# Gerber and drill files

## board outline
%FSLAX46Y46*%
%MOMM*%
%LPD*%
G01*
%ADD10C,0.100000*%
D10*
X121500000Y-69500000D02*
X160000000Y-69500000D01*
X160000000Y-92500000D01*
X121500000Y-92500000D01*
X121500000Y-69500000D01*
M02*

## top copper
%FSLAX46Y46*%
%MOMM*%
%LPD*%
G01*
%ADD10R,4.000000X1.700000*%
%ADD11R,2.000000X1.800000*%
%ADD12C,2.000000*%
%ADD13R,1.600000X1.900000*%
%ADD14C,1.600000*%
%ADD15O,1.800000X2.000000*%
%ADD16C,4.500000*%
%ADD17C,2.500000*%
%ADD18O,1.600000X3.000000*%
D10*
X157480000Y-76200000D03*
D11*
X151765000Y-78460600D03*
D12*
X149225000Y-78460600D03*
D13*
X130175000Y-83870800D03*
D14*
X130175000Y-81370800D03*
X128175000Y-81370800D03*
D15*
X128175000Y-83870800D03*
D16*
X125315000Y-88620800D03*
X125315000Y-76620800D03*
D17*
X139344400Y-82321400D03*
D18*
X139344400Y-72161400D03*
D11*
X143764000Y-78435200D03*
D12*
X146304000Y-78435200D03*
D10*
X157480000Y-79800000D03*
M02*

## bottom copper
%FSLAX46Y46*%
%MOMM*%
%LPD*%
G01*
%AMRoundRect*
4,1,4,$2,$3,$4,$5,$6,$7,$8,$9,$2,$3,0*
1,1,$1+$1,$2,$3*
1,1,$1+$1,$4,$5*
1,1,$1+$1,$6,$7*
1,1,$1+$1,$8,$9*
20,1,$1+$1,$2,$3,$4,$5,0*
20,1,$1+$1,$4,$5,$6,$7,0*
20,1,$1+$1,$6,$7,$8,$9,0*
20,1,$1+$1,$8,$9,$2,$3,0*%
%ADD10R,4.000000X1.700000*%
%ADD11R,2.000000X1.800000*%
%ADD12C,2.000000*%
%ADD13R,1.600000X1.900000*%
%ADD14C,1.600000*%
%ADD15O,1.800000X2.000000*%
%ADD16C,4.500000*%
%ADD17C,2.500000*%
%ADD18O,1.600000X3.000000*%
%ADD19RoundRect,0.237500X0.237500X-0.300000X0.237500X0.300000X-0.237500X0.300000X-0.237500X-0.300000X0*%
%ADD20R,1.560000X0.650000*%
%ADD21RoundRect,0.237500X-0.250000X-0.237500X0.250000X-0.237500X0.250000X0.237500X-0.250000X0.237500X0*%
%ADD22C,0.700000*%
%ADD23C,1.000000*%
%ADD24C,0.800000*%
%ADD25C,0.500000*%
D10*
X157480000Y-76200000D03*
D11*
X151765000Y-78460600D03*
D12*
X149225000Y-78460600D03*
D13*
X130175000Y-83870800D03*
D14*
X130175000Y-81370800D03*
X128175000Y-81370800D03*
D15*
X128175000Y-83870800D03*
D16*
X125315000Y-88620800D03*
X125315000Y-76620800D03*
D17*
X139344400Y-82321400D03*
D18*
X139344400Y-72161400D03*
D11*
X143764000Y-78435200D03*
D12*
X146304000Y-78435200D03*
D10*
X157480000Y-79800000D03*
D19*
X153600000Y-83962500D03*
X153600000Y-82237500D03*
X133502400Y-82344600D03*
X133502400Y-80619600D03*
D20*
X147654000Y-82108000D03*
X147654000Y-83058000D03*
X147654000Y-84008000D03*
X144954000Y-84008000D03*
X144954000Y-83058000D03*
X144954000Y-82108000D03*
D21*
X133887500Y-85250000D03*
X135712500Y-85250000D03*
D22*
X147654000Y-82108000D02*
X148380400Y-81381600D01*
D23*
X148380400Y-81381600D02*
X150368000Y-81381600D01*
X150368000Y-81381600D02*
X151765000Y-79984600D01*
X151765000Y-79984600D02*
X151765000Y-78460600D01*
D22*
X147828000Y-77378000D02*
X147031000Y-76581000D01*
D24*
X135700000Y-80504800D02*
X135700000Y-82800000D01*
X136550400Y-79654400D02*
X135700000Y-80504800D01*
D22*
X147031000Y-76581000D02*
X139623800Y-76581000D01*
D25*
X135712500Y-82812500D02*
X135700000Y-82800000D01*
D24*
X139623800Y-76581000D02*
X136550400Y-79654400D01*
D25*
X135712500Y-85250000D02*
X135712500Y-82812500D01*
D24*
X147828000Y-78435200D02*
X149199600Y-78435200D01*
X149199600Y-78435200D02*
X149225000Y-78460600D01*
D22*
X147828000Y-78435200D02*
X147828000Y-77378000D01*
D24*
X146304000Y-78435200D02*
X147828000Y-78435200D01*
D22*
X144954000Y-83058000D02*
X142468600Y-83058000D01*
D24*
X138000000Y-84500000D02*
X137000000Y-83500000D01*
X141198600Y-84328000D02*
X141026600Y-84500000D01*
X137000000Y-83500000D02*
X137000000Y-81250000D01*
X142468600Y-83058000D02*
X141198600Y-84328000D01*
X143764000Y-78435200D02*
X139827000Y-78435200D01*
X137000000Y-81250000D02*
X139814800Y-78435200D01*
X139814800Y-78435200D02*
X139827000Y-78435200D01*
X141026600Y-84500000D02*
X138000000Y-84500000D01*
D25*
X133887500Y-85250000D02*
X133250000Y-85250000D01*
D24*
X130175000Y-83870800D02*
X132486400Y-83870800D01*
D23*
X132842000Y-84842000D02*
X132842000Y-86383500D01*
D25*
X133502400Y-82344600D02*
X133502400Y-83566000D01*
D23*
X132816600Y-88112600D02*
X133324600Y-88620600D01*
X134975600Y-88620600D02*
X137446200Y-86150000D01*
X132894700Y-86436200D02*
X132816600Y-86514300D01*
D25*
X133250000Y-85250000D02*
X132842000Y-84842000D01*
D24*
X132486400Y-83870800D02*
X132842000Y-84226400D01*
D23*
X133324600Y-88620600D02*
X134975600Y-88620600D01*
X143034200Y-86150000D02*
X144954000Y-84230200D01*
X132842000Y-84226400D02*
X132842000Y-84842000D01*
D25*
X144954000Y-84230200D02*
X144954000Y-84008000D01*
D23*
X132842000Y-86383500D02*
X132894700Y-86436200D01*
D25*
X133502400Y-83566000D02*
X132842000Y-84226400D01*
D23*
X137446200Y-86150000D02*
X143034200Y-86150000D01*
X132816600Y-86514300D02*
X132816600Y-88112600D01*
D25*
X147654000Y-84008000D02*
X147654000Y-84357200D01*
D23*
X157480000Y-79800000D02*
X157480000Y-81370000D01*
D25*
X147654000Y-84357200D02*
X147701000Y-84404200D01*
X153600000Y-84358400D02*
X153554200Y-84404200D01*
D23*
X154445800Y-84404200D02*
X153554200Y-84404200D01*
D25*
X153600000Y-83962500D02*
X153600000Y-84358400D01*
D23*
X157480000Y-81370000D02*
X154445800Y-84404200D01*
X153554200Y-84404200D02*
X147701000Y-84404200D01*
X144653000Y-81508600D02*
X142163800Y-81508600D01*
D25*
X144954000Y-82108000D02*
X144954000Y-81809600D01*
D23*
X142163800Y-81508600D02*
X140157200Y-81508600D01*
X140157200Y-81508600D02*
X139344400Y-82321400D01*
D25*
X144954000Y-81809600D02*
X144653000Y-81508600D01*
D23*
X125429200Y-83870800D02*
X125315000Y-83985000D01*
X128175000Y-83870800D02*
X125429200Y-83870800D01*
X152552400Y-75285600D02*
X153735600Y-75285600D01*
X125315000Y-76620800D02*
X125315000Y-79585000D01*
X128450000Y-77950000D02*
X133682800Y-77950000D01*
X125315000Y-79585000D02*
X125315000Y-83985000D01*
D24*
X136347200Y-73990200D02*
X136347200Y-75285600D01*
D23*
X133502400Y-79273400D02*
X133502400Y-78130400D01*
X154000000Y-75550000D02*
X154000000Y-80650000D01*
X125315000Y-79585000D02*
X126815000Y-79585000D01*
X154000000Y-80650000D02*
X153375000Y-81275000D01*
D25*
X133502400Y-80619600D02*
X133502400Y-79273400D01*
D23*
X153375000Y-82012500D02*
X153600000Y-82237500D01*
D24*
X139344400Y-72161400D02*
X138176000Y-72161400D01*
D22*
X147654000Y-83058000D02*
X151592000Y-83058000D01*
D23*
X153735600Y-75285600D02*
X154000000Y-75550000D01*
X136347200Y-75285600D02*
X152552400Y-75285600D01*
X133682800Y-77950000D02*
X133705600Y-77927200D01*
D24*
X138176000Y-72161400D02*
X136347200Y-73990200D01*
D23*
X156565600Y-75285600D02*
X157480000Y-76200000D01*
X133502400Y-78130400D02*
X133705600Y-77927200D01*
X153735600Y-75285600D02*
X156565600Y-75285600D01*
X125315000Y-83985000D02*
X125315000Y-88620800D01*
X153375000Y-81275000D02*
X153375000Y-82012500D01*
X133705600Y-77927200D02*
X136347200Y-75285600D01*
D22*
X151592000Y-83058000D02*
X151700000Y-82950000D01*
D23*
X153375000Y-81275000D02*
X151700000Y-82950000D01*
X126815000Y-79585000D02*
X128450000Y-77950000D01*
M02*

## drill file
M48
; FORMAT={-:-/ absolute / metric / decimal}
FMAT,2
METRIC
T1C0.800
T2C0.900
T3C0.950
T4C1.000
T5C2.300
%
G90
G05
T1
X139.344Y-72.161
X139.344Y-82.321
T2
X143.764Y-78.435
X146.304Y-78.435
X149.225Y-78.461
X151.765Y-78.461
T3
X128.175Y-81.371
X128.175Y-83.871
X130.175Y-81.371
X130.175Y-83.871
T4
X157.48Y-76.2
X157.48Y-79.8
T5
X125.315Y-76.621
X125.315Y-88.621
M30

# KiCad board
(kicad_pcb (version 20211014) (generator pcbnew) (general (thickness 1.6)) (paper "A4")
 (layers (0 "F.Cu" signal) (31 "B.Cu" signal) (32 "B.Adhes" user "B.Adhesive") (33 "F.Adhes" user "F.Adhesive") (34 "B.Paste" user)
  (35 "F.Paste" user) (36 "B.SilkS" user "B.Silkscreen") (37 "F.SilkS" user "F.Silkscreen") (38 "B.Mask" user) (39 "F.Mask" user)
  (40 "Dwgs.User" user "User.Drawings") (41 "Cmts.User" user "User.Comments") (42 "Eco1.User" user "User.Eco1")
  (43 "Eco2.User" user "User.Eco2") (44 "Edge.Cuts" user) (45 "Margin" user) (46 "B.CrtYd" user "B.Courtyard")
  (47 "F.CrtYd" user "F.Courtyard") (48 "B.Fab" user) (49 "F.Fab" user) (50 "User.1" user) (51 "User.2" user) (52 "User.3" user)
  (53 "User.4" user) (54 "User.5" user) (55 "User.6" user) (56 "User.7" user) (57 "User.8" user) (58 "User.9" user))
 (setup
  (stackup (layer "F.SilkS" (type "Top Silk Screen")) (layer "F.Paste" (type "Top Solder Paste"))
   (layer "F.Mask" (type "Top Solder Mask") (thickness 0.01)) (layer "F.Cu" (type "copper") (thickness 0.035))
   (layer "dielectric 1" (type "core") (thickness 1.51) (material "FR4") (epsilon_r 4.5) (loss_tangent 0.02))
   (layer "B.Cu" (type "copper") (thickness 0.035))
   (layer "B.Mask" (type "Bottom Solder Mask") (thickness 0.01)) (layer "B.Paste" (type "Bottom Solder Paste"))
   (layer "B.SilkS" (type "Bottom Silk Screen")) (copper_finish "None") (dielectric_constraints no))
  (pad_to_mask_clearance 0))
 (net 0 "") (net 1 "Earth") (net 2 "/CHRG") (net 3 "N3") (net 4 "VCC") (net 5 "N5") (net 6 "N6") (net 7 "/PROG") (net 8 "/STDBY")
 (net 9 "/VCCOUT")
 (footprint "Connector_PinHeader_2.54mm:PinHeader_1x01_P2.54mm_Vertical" (layer "F.Cu") (at 157.48 76.2)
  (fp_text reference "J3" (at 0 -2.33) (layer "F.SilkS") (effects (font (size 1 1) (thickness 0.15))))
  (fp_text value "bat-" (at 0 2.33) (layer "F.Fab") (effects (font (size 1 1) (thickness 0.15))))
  (pad "1" thru_hole rect (at 0 0) (size 4 1.7) (drill 1) (layers *.Cu) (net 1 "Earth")))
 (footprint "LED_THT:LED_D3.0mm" (layer "F.Cu") (at 151.765 78.4606 180)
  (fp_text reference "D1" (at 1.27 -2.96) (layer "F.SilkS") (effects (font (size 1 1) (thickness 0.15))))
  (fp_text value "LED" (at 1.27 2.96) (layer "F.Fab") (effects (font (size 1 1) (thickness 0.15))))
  (pad "1" thru_hole rect (at 0 0 180) (size 2 1.8) (drill 0.9) (layers *.Cu *.Mask) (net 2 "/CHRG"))
  (pad "2" thru_hole circle (at 2.54 0 180) (size 2 2) (drill 0.9) (layers *.Cu *.Mask) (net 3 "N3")))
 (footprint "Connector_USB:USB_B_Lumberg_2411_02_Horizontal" (layer "F.Cu") (at 130.175 83.8708 180)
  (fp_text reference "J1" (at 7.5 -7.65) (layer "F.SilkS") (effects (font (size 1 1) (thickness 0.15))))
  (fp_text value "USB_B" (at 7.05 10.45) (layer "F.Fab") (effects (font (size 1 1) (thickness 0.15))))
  (pad "1" thru_hole rect (at 0 0 270) (size 1.9 1.6) (drill 0.95) (layers *.Cu *.Mask) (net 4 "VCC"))
  (pad "2" thru_hole circle (at 0 2.5 270) (size 1.6 1.6) (drill 0.95) (layers *.Cu *.Mask) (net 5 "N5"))
  (pad "3" thru_hole circle (at 2 2.5 270) (size 1.6 1.6) (drill 0.95) (layers *.Cu *.Mask) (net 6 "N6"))
  (pad "4" thru_hole oval (at 2 0 270) (size 2 1.8) (drill 0.95) (layers *.Cu *.Mask) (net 1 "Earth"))
  (pad "5" thru_hole circle (at 4.86 -4.75 270) (size 4.5 4.5) (drill 2.3) (layers *.Cu *.Mask) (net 1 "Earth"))
  (pad "5" thru_hole circle (at 4.86 7.25 270) (size 4.5 4.5) (drill 2.3) (layers *.Cu *.Mask) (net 1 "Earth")))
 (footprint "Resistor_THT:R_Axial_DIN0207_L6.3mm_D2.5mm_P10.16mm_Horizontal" (layer "F.Cu") (at 139.3444 82.3214 90)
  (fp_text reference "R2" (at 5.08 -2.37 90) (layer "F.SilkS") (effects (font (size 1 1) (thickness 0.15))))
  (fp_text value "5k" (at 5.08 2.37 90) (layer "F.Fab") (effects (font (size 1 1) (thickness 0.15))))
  (pad "1" thru_hole circle (at 0 0 90) (size 2.5 2.5) (drill 0.8) (layers *.Cu *.Mask) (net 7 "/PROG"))
  (pad "2" thru_hole oval (at 10.16 0 90) (size 3 1.6) (drill 0.8) (layers *.Cu *.Mask) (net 1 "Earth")))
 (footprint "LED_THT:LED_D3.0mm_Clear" (layer "F.Cu") (at 143.764 78.4352)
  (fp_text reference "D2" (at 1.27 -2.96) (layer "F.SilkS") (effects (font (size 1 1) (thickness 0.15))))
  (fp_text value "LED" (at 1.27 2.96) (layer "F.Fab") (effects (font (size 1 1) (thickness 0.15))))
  (pad "1" thru_hole rect (at 0 0) (size 2 1.8) (drill 0.9) (layers *.Cu *.Mask) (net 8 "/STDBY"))
  (pad "2" thru_hole circle (at 2.54 0) (size 2 2) (drill 0.9) (layers *.Cu *.Mask) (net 3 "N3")))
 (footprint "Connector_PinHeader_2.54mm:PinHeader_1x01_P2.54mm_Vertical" (layer "F.Cu") (at 157.48 79.8)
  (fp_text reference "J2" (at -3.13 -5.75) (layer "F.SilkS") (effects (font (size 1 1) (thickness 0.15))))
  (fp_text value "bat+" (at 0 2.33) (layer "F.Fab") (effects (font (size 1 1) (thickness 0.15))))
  (pad "1" thru_hole rect (at 0 0) (size 4 1.7) (drill 1) (layers *.Cu) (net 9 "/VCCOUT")))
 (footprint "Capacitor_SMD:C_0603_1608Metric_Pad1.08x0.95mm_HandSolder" (layer "B.Cu") (at 153.6 83.1 90)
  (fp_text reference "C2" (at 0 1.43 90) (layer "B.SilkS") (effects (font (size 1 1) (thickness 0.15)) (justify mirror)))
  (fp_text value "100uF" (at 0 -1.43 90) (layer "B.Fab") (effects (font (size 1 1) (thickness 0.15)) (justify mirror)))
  (pad "1" smd roundrect (at -0.8625 0 90) (size 1.075 0.95) (layers "B.Cu" "B.Paste" "B.Mask") (roundrect_rratio 0.25) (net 9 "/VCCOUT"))
  (pad "2" smd roundrect (at 0.8625 0 90) (size 1.075 0.95) (layers "B.Cu" "B.Paste" "B.Mask") (roundrect_rratio 0.25) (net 1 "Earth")))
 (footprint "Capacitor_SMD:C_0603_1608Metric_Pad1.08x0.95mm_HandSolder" (layer "B.Cu") (at 133.5024 81.4821 90)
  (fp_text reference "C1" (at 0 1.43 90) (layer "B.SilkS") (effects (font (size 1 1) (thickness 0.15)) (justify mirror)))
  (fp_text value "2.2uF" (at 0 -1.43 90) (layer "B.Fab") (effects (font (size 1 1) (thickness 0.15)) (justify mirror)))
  (pad "1" smd roundrect (at -0.8625 0 90) (size 1.075 0.95) (layers "B.Cu" "B.Paste" "B.Mask") (roundrect_rratio 0.25) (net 4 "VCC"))
  (pad "2" smd roundrect (at 0.8625 0 90) (size 1.075 0.95) (layers "B.Cu" "B.Paste" "B.Mask") (roundrect_rratio 0.25) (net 1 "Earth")))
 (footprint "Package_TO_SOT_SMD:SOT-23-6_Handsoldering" (layer "B.Cu") (at 146.304 83.058 180)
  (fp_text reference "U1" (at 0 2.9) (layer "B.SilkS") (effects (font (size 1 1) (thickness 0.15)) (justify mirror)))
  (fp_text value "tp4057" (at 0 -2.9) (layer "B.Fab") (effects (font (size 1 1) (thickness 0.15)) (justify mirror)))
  (pad "1" smd rect (at -1.35 0.95 180) (size 1.56 0.65) (layers "B.Cu" "B.Paste" "B.Mask") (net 2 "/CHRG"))
  (pad "2" smd rect (at -1.35 0 180) (size 1.56 0.65) (layers "B.Cu" "B.Paste" "B.Mask") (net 1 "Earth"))
  (pad "3" smd rect (at -1.35 -0.95 180) (size 1.56 0.65) (layers "B.Cu" "B.Paste" "B.Mask") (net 9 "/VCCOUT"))
  (pad "4" smd rect (at 1.35 -0.95 180) (size 1.56 0.65) (layers "B.Cu" "B.Paste" "B.Mask") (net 4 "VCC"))
  (pad "5" smd rect (at 1.35 0 180) (size 1.56 0.65) (layers "B.Cu" "B.Paste" "B.Mask") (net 8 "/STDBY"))
  (pad "6" smd rect (at 1.35 0.95 180) (size 1.56 0.65) (layers "B.Cu" "B.Paste" "B.Mask") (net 7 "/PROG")))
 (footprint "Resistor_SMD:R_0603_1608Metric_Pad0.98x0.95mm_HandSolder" (layer "B.Cu") (at 134.8 85.25)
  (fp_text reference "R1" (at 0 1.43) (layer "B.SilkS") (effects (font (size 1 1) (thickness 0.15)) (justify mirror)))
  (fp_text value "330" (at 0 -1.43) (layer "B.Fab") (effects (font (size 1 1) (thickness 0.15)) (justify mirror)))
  (pad "1" smd roundrect (at -0.9125 0) (size 0.975 0.95) (layers "B.Cu" "B.Paste" "B.Mask") (roundrect_rratio 0.25) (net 4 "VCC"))
  (pad "2" smd roundrect (at 0.9125 0) (size 0.975 0.95) (layers "B.Cu" "B.Paste" "B.Mask") (roundrect_rratio 0.25) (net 3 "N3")))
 (gr_rect (start 121.5 69.5) (end 160 92.5) (layer "Edge.Cuts") (width 0.1) (fill none))
 (segment (start 147.654 82.108) (end 148.3804 81.3816) (width 0.7) (layer "B.Cu") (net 2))
 (segment (start 148.3804 81.3816) (end 150.368 81.3816) (width 1) (layer "B.Cu") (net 2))
 (segment (start 150.368 81.3816) (end 151.765 79.9846) (width 1) (layer "B.Cu") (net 2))
 (segment (start 151.765 79.9846) (end 151.765 78.4606) (width 1) (layer "B.Cu") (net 2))
 (segment (start 147.828 77.378) (end 147.031 76.581) (width 0.7) (layer "B.Cu") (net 3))
 (segment (start 135.7 80.5048) (end 135.7 82.8) (width 0.8) (layer "B.Cu") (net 3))
 (segment (start 136.5504 79.6544) (end 135.7 80.5048) (width 0.8) (layer "B.Cu") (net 3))
 (segment (start 147.031 76.581) (end 139.6238 76.581) (width 0.7) (layer "B.Cu") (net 3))
 (segment (start 135.7125 82.8125) (end 135.7 82.8) (width 0.5) (layer "B.Cu") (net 3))
 (segment (start 139.6238 76.581) (end 136.5504 79.6544) (width 0.8) (layer "B.Cu") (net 3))
 (segment (start 135.7125 85.25) (end 135.7125 82.8125) (width 0.5) (layer "B.Cu") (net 3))
 (segment (start 147.828 78.4352) (end 149.1996 78.4352) (width 0.8) (layer "B.Cu") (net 3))
 (segment (start 149.1996 78.4352) (end 149.225 78.4606) (width 0.8) (layer "B.Cu") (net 3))
 (segment (start 147.828 78.4352) (end 147.828 77.378) (width 0.7) (layer "B.Cu") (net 3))
 (segment (start 146.304 78.4352) (end 147.828 78.4352) (width 0.8) (layer "B.Cu") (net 3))
 (segment (start 144.954 83.058) (end 142.4686 83.058) (width 0.7) (layer "B.Cu") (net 8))
 (segment (start 138 84.5) (end 137 83.5) (width 0.8) (layer "B.Cu") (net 8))
 (segment (start 141.1986 84.328) (end 141.0266 84.5) (width 0.8) (layer "B.Cu") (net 8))
 (segment (start 137 83.5) (end 137 81.25) (width 0.8) (layer "B.Cu") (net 8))
 (segment (start 142.4686 83.058) (end 141.1986 84.328) (width 0.8) (layer "B.Cu") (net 8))
 (segment (start 143.764 78.4352) (end 139.827 78.4352) (width 0.8) (layer "B.Cu") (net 8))
 (segment (start 137 81.25) (end 139.8148 78.4352) (width 0.8) (layer "B.Cu") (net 8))
 (segment (start 139.8148 78.4352) (end 139.827 78.4352) (width 0.8) (layer "B.Cu") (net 8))
 (segment (start 141.0266 84.5) (end 138 84.5) (width 0.8) (layer "B.Cu") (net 8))
 (segment (start 133.8875 85.25) (end 133.25 85.25) (width 0.5) (layer "B.Cu") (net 4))
 (segment (start 130.175 83.8708) (end 132.4864 83.8708) (width 0.8) (layer "B.Cu") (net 4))
 (segment (start 132.842 84.842) (end 132.842 86.3835) (width 1) (layer "B.Cu") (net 4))
 (segment (start 133.5024 82.3446) (end 133.5024 83.566) (width 0.5) (layer "B.Cu") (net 4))
 (segment (start 132.8166 88.1126) (end 133.3246 88.6206) (width 1) (layer "B.Cu") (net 4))
 (segment (start 134.9756 88.6206) (end 137.4462 86.15) (width 1) (layer "B.Cu") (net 4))
 (segment (start 132.8947 86.4362) (end 132.8166 86.5143) (width 1) (layer "B.Cu") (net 4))
 (segment (start 133.25 85.25) (end 132.842 84.842) (width 0.5) (layer "B.Cu") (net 4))
 (segment (start 132.4864 83.8708) (end 132.842 84.2264) (width 0.8) (layer "B.Cu") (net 4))
 (segment (start 133.3246 88.6206) (end 134.9756 88.6206) (width 1) (layer "B.Cu") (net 4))
 (segment (start 143.0342 86.15) (end 144.954 84.2302) (width 1) (layer "B.Cu") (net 4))
 (segment (start 132.842 84.2264) (end 132.842 84.842) (width 1) (layer "B.Cu") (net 4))
 (segment (start 144.954 84.2302) (end 144.954 84.008) (width 0.5) (layer "B.Cu") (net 4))
 (segment (start 132.842 86.3835) (end 132.8947 86.4362) (width 1) (layer "B.Cu") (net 4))
 (segment (start 133.5024 83.566) (end 132.842 84.2264) (width 0.5) (layer "B.Cu") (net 4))
 (segment (start 137.4462 86.15) (end 143.0342 86.15) (width 1) (layer "B.Cu") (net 4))
 (segment (start 132.8166 86.5143) (end 132.8166 88.1126) (width 1) (layer "B.Cu") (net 4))
 (segment (start 147.654 84.008) (end 147.654 84.3572) (width 0.5) (layer "B.Cu") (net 9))
 (segment (start 157.48 79.8) (end 157.48 81.37) (width 1) (layer "B.Cu") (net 9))
 (segment (start 147.654 84.3572) (end 147.701 84.4042) (width 0.5) (layer "B.Cu") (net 9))
 (segment (start 153.6 84.3584) (end 153.5542 84.4042) (width 0.5) (layer "B.Cu") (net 9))
 (segment (start 154.4458 84.4042) (end 153.5542 84.4042) (width 1) (layer "B.Cu") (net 9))
 (segment (start 153.6 83.9625) (end 153.6 84.3584) (width 0.5) (layer "B.Cu") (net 9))
 (segment (start 157.48 81.37) (end 154.4458 84.4042) (width 1) (layer "B.Cu") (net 9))
 (segment (start 153.5542 84.4042) (end 147.701 84.4042) (width 1) (layer "B.Cu") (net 9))
 (segment (start 144.653 81.5086) (end 142.1638 81.5086) (width 1) (layer "B.Cu") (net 7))
 (segment (start 144.954 82.108) (end 144.954 81.8096) (width 0.5) (layer "B.Cu") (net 7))
 (segment (start 142.1638 81.5086) (end 140.1572 81.5086) (width 1) (layer "B.Cu") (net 7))
 (segment (start 140.1572 81.5086) (end 139.3444 82.3214) (width 1) (layer "B.Cu") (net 7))
 (segment (start 144.954 81.8096) (end 144.653 81.5086) (width 0.5) (layer "B.Cu") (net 7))
 (segment (start 125.4292 83.8708) (end 125.315 83.985) (width 1) (layer "B.Cu") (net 1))
 (segment (start 128.175 83.8708) (end 125.4292 83.8708) (width 1) (layer "B.Cu") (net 1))
 (segment (start 152.5524 75.2856) (end 153.7356 75.2856) (width 1) (layer "B.Cu") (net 1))
 (segment (start 125.315 76.6208) (end 125.315 79.585) (width 1) (layer "B.Cu") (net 1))
 (segment (start 128.45 77.95) (end 133.6828 77.95) (width 1) (layer "B.Cu") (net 1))
 (segment (start 125.315 79.585) (end 125.315 83.985) (width 1) (layer "B.Cu") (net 1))
 (segment (start 136.3472 73.9902) (end 136.3472 75.2856) (width 0.8) (layer "B.Cu") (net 1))
 (segment (start 133.5024 79.2734) (end 133.5024 78.1304) (width 1) (layer "B.Cu") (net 1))
 (segment (start 154 75.55) (end 154 80.65) (width 1) (layer "B.Cu") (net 1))
 (segment (start 125.315 79.585) (end 126.815 79.585) (width 1) (layer "B.Cu") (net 1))
 (segment (start 154 80.65) (end 153.375 81.275) (width 1) (layer "B.Cu") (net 1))
 (segment (start 133.5024 80.6196) (end 133.5024 79.2734) (width 0.5) (layer "B.Cu") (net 1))
 (segment (start 153.375 82.0125) (end 153.6 82.2375) (width 1) (layer "B.Cu") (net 1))
 (segment (start 139.3444 72.1614) (end 138.176 72.1614) (width 0.8) (layer "B.Cu") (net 1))
 (segment (start 147.654 83.058) (end 151.592 83.058) (width 0.7) (layer "B.Cu") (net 1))
 (segment (start 153.7356 75.2856) (end 154 75.55) (width 1) (layer "B.Cu") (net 1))
 (segment (start 136.3472 75.2856) (end 152.5524 75.2856) (width 1) (layer "B.Cu") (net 1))
 (segment (start 133.6828 77.95) (end 133.7056 77.9272) (width 1) (layer "B.Cu") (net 1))
 (segment (start 138.176 72.1614) (end 136.3472 73.9902) (width 0.8) (layer "B.Cu") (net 1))
 (segment (start 156.5656 75.2856) (end 157.48 76.2) (width 1) (layer "B.Cu") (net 1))
 (segment (start 133.5024 78.1304) (end 133.7056 77.9272) (width 1) (layer "B.Cu") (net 1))
 (segment (start 153.7356 75.2856) (end 156.5656 75.2856) (width 1) (layer "B.Cu") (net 1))
 (segment (start 125.315 83.985) (end 125.315 88.6208) (width 1) (layer "B.Cu") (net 1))
 (segment (start 153.375 81.275) (end 153.375 82.0125) (width 1) (layer "B.Cu") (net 1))
 (segment (start 133.7056 77.9272) (end 136.3472 75.2856) (width 1) (layer "B.Cu") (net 1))
 (segment (start 151.592 83.058) (end 151.7 82.95) (width 0.7) (layer "B.Cu") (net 1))
 (segment (start 153.375 81.275) (end 151.7 82.95) (width 1) (layer "B.Cu") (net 1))
 (segment (start 126.815 79.585) (end 128.45 77.95) (width 1) (layer "B.Cu") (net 1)))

